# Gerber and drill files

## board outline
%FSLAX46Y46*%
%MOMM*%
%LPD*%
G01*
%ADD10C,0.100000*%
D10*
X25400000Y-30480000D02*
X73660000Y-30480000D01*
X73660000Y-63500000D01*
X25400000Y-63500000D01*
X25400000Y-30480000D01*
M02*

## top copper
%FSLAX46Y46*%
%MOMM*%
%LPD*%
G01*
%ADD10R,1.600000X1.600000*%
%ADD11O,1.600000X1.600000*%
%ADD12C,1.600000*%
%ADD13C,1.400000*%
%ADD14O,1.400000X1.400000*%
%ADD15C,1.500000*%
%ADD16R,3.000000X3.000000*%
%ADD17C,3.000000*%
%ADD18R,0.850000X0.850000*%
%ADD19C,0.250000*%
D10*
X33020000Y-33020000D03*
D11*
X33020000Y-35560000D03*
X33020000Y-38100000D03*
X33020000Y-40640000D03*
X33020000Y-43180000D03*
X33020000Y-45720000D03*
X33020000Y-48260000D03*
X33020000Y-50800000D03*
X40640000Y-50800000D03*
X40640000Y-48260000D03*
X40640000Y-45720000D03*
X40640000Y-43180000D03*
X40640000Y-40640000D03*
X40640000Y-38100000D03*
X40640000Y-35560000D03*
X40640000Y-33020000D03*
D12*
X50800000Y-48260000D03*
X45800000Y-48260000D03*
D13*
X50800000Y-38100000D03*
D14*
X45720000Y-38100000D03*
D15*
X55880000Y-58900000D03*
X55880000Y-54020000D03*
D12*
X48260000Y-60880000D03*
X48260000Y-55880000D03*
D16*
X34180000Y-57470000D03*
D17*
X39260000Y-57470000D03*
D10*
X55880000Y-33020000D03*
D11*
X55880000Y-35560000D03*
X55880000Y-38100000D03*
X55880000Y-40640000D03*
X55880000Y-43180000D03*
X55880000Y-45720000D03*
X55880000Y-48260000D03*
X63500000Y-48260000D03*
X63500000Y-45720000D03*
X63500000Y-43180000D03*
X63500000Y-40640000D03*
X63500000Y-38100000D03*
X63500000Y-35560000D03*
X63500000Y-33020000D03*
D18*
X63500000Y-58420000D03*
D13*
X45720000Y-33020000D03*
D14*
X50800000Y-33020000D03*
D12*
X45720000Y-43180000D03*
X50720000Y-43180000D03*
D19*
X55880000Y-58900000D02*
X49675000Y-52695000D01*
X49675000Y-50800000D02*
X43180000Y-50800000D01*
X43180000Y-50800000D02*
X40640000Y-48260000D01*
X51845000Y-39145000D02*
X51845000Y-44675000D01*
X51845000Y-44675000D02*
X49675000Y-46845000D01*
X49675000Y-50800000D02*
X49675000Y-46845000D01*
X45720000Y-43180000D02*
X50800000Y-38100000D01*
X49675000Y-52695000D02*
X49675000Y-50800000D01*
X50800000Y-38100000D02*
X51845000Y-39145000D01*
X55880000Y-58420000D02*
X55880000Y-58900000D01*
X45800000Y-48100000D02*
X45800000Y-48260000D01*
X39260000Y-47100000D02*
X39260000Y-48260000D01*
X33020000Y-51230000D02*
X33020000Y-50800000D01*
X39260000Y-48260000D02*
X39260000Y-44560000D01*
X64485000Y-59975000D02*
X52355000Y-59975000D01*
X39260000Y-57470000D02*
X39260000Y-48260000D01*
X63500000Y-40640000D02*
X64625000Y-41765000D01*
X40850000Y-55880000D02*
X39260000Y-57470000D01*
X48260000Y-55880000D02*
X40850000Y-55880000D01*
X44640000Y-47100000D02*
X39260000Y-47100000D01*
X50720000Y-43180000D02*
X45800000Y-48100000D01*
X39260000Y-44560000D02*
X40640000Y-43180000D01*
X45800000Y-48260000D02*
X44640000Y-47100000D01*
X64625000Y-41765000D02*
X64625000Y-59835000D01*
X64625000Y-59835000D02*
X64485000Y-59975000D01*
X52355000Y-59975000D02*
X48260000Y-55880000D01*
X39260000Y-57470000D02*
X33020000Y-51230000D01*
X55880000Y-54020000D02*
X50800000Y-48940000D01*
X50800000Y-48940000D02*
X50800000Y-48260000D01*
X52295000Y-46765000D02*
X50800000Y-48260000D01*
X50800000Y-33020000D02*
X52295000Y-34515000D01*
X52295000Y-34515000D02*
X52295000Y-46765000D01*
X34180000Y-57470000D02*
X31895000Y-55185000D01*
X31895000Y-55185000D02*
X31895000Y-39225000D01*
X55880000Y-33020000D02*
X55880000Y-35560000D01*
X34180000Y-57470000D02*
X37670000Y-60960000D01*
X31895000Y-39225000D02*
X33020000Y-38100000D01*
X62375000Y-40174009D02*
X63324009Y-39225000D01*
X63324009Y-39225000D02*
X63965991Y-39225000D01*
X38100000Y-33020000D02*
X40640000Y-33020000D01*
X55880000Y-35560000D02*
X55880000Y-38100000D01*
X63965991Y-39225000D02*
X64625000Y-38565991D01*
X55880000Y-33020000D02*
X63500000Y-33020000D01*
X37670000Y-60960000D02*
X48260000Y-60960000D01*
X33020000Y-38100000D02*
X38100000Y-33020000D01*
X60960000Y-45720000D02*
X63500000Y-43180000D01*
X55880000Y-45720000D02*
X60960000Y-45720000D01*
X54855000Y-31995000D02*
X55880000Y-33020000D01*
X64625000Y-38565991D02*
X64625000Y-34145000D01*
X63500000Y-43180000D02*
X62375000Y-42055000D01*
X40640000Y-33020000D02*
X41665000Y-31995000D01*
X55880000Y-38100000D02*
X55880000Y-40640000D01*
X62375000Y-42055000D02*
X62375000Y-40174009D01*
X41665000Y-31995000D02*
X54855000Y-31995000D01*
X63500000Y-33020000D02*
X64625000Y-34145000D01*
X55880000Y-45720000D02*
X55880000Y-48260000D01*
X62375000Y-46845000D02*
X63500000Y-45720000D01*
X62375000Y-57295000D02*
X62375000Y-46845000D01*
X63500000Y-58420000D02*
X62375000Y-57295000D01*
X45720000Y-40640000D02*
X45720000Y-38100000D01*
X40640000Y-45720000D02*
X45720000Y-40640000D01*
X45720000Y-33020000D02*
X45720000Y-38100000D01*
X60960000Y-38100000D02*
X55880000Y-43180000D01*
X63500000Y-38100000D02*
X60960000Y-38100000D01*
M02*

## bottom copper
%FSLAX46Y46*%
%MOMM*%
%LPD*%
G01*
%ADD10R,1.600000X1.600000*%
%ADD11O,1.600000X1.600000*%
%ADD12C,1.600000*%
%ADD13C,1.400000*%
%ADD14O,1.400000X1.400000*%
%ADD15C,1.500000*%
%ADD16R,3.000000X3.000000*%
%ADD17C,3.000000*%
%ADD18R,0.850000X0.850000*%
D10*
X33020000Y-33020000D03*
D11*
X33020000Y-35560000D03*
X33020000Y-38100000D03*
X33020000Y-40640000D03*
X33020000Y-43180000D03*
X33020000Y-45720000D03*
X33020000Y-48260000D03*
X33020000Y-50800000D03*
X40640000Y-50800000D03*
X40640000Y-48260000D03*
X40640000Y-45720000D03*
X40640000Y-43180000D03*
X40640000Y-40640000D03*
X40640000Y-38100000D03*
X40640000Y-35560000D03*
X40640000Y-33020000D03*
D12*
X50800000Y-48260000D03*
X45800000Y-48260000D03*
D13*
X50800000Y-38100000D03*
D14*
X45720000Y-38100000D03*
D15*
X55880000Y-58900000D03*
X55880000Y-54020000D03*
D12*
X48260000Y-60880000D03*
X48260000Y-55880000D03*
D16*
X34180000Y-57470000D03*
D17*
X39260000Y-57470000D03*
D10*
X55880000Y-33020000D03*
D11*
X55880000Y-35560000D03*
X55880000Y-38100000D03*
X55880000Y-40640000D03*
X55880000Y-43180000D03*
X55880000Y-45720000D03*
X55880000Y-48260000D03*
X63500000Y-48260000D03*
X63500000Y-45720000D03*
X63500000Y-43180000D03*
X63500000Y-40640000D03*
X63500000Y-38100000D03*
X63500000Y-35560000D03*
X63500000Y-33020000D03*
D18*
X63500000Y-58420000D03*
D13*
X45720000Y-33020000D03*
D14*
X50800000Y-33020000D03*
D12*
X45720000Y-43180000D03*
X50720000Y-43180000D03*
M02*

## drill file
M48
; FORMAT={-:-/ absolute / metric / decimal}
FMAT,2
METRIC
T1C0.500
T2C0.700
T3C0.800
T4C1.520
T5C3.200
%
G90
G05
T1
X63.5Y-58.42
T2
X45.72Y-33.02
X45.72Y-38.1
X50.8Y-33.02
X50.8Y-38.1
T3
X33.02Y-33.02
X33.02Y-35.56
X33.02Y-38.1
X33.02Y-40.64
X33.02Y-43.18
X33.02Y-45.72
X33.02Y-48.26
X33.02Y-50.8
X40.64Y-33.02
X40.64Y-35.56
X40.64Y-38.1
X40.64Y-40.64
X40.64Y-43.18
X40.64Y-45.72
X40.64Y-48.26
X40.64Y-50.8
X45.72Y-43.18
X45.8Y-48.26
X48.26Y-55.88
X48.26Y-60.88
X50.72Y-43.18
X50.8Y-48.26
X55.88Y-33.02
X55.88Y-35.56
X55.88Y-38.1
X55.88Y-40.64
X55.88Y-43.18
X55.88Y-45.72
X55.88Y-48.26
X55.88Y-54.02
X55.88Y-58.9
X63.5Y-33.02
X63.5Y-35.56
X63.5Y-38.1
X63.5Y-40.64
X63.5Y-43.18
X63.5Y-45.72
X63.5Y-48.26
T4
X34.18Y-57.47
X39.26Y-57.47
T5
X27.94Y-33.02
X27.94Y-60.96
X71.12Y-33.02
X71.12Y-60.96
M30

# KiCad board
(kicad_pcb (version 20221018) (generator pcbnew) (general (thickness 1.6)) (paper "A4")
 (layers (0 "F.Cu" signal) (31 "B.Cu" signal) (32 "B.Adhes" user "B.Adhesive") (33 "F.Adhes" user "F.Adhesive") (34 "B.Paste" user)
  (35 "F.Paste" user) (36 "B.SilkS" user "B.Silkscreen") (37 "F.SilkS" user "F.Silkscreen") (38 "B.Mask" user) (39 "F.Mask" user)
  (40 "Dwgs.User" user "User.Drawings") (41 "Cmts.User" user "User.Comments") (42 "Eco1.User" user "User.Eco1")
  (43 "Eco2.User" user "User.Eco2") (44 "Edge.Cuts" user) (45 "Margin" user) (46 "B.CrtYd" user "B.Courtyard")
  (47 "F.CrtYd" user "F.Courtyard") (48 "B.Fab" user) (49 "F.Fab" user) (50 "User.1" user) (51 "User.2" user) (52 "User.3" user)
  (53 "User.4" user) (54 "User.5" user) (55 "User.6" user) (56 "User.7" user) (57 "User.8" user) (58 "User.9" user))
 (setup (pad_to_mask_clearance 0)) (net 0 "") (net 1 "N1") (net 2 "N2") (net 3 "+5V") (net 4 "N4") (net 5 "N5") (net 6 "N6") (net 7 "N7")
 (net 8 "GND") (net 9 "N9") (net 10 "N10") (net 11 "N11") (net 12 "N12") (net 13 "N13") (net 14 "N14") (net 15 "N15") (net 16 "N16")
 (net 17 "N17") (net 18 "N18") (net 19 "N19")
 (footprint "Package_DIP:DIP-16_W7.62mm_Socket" (layer "F.Cu") (at 33.02 33.02)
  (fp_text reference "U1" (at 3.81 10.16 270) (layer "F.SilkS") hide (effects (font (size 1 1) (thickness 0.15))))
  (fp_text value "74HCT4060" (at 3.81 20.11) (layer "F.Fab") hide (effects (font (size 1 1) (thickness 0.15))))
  (pad "1" thru_hole rect (at 0 0) (size 1.6 1.6) (drill 0.8) (layers "*.Cu" "*.Mask") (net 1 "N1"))
  (pad "2" thru_hole oval (at 0 2.54) (size 1.6 1.6) (drill 0.8) (layers "*.Cu" "*.Mask") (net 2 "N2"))
  (pad "3" thru_hole oval (at 0 5.08) (size 1.6 1.6) (drill 0.8) (layers "*.Cu" "*.Mask") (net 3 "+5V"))
  (pad "4" thru_hole oval (at 0 7.62) (size 1.6 1.6) (drill 0.8) (layers "*.Cu" "*.Mask") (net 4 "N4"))
  (pad "5" thru_hole oval (at 0 10.16) (size 1.6 1.6) (drill 0.8) (layers "*.Cu" "*.Mask") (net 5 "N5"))
  (pad "6" thru_hole oval (at 0 12.7) (size 1.6 1.6) (drill 0.8) (layers "*.Cu" "*.Mask") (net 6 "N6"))
  (pad "7" thru_hole oval (at 0 15.24) (size 1.6 1.6) (drill 0.8) (layers "*.Cu" "*.Mask") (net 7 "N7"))
  (pad "8" thru_hole oval (at 0 17.78) (size 1.6 1.6) (drill 0.8) (layers "*.Cu" "*.Mask") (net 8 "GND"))
  (pad "9" thru_hole oval (at 7.62 17.78) (size 1.6 1.6) (drill 0.8) (layers "*.Cu" "*.Mask") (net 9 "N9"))
  (pad "10" thru_hole oval (at 7.62 15.24) (size 1.6 1.6) (drill 0.8) (layers "*.Cu" "*.Mask") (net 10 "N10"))
  (pad "11" thru_hole oval (at 7.62 12.7) (size 1.6 1.6) (drill 0.8) (layers "*.Cu" "*.Mask") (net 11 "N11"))
  (pad "12" thru_hole oval (at 7.62 10.16) (size 1.6 1.6) (drill 0.8) (layers "*.Cu" "*.Mask") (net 8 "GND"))
  (pad "13" thru_hole oval (at 7.62 7.62) (size 1.6 1.6) (drill 0.8) (layers "*.Cu" "*.Mask") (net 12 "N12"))
  (pad "14" thru_hole oval (at 7.62 5.08) (size 1.6 1.6) (drill 0.8) (layers "*.Cu" "*.Mask") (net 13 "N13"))
  (pad "15" thru_hole oval (at 7.62 2.54) (size 1.6 1.6) (drill 0.8) (layers "*.Cu" "*.Mask") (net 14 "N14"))
  (pad "16" thru_hole oval (at 7.62 0) (size 1.6 1.6) (drill 0.8) (layers "*.Cu" "*.Mask") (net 3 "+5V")))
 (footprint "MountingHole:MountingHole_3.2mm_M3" (layer "F.Cu") (at 71.12 60.96)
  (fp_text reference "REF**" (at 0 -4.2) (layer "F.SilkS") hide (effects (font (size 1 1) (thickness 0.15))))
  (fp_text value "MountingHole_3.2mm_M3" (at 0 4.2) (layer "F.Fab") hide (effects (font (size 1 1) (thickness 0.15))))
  (pad "" np_thru_hole circle (at 0 0) (size 3.2 3.2) (drill 3.2) (layers "*.Cu" "*.Mask")))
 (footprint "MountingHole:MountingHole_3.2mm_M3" (layer "F.Cu") (at 27.94 60.96)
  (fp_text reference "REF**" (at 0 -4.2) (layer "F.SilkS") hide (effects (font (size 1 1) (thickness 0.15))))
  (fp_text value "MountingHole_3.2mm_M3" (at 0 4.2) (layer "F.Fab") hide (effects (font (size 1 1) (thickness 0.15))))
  (pad "" np_thru_hole circle (at 0 0) (size 3.2 3.2) (drill 3.2) (layers "*.Cu" "*.Mask")))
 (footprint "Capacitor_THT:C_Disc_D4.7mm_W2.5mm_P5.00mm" (layer "F.Cu") (at 50.8 48.26 180)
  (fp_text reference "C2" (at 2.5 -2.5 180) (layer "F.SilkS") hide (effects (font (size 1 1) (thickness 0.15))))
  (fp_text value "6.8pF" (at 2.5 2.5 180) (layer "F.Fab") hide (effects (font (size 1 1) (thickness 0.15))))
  (pad "1" thru_hole circle (at 0 0 180) (size 1.6 1.6) (drill 0.8) (layers "*.Cu" "*.Mask") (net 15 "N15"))
  (pad "2" thru_hole circle (at 5 0 180) (size 1.6 1.6) (drill 0.8) (layers "*.Cu" "*.Mask") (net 8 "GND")))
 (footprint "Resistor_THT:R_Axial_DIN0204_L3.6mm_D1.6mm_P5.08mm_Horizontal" (layer "F.Cu") (at 50.8 38.1 180)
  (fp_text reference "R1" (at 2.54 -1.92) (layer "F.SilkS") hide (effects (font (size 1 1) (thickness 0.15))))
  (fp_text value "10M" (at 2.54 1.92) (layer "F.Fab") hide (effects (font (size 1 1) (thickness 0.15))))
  (pad "1" thru_hole circle (at 0 0 180) (size 1.4 1.4) (drill 0.7) (layers "*.Cu" "*.Mask") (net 10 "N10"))
  (pad "2" thru_hole oval (at 5.08 0 180) (size 1.4 1.4) (drill 0.7) (layers "*.Cu" "*.Mask") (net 11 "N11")))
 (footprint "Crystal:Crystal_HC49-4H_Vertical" (layer "F.Cu") (at 55.88 58.9 90)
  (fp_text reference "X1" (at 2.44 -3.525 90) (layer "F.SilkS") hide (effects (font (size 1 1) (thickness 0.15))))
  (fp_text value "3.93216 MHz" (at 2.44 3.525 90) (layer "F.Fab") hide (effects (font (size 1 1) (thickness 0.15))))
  (pad "1" thru_hole circle (at 0 0 90) (size 1.5 1.5) (drill 0.8) (layers "*.Cu" "*.Mask") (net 10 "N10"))
  (pad "2" thru_hole circle (at 4.88 0 90) (size 1.5 1.5) (drill 0.8) (layers "*.Cu" "*.Mask") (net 15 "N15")))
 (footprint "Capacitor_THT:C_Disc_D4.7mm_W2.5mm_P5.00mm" (layer "F.Cu") (at 48.26 60.88 90)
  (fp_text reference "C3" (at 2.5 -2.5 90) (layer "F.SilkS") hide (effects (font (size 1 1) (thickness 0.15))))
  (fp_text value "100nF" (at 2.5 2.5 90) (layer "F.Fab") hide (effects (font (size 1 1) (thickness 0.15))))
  (pad "1" thru_hole circle (at 0 0 90) (size 1.6 1.6) (drill 0.8) (layers "*.Cu" "*.Mask") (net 3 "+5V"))
  (pad "2" thru_hole circle (at 5 0 90) (size 1.6 1.6) (drill 0.8) (layers "*.Cu" "*.Mask") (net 8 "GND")))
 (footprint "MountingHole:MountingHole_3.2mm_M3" (layer "F.Cu") (at 71.12 33.02)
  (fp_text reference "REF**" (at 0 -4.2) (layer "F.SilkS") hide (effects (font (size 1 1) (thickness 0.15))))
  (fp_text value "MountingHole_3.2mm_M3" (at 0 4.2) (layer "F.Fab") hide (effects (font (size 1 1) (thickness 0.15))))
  (pad "" np_thru_hole circle (at 0 0) (size 3.2 3.2) (drill 3.2) (layers "*.Cu" "*.Mask")))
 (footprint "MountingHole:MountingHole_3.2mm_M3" (layer "F.Cu") (at 27.94 33.02)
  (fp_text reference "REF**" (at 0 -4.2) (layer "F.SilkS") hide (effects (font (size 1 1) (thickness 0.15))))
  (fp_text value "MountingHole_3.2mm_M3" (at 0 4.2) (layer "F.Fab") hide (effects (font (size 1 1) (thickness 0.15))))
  (pad "" np_thru_hole circle (at 0 0) (size 3.2 3.2) (drill 3.2) (layers "*.Cu" "*.Mask")))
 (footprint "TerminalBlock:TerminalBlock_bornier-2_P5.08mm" (layer "F.Cu") (at 34.18 57.47)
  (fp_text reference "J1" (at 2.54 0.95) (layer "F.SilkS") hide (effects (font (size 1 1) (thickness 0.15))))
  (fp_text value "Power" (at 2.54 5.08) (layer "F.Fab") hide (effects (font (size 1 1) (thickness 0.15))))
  (pad "1" thru_hole rect (at 0 0) (size 3 3) (drill 1.52) (layers "*.Cu" "*.Mask") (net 3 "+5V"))
  (pad "2" thru_hole circle (at 5.08 0) (size 3 3) (drill 1.52) (layers "*.Cu" "*.Mask") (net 8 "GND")))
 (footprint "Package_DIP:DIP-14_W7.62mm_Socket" (layer "F.Cu") (at 55.88 33.02)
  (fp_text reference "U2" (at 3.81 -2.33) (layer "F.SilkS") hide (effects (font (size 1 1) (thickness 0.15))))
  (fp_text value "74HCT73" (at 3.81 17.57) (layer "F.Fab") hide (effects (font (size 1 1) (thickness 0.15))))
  (pad "1" thru_hole rect (at 0 0) (size 1.6 1.6) (drill 0.8) (layers "*.Cu" "*.Mask") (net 3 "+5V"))
  (pad "2" thru_hole oval (at 0 2.54) (size 1.6 1.6) (drill 0.8) (layers "*.Cu" "*.Mask") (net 3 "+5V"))
  (pad "3" thru_hole oval (at 0 5.08) (size 1.6 1.6) (drill 0.8) (layers "*.Cu" "*.Mask") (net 3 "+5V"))
  (pad "4" thru_hole oval (at 0 7.62) (size 1.6 1.6) (drill 0.8) (layers "*.Cu" "*.Mask") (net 3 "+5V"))
  (pad "5" thru_hole oval (at 0 10.16) (size 1.6 1.6) (drill 0.8) (layers "*.Cu" "*.Mask") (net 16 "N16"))
  (pad "6" thru_hole oval (at 0 12.7) (size 1.6 1.6) (drill 0.8) (layers "*.Cu" "*.Mask") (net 3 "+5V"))
  (pad "7" thru_hole oval (at 0 15.24) (size 1.6 1.6) (drill 0.8) (layers "*.Cu" "*.Mask") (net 3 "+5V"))
  (pad "8" thru_hole oval (at 7.62 15.24) (size 1.6 1.6) (drill 0.8) (layers "*.Cu" "*.Mask") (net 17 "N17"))
  (pad "9" thru_hole oval (at 7.62 12.7) (size 1.6 1.6) (drill 0.8) (layers "*.Cu" "*.Mask") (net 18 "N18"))
  (pad "10" thru_hole oval (at 7.62 10.16) (size 1.6 1.6) (drill 0.8) (layers "*.Cu" "*.Mask") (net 3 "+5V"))
  (pad "11" thru_hole oval (at 7.62 7.62) (size 1.6 1.6) (drill 0.8) (layers "*.Cu" "*.Mask") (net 8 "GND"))
  (pad "12" thru_hole oval (at 7.62 5.08) (size 1.6 1.6) (drill 0.8) (layers "*.Cu" "*.Mask") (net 16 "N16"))
  (pad "13" thru_hole oval (at 7.62 2.54) (size 1.6 1.6) (drill 0.8) (layers "*.Cu" "*.Mask") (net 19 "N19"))
  (pad "14" thru_hole oval (at 7.62 0) (size 1.6 1.6) (drill 0.8) (layers "*.Cu" "*.Mask") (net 3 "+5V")))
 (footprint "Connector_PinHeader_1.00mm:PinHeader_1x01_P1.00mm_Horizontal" (layer "F.Cu") (at 63.5 58.42 -90)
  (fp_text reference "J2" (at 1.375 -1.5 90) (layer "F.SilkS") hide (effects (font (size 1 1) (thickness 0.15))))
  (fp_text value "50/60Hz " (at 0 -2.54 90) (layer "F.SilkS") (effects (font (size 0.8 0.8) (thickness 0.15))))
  (pad "1" thru_hole rect (at 0 0 270) (size 0.85 0.85) (drill 0.5) (layers "*.Cu" "*.Mask") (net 18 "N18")))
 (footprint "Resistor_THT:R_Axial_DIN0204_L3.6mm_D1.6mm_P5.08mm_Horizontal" (layer "F.Cu") (at 45.72 33.02)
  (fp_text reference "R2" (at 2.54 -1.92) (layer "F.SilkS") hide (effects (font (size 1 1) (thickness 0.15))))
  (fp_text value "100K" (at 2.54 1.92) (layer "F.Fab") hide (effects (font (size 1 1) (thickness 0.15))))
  (pad "1" thru_hole circle (at 0 0) (size 1.4 1.4) (drill 0.7) (layers "*.Cu" "*.Mask") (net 11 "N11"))
  (pad "2" thru_hole oval (at 5.08 0) (size 1.4 1.4) (drill 0.7) (layers "*.Cu" "*.Mask") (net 15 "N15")))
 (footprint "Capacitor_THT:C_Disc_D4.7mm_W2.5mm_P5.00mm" (layer "F.Cu") (at 45.72 43.18)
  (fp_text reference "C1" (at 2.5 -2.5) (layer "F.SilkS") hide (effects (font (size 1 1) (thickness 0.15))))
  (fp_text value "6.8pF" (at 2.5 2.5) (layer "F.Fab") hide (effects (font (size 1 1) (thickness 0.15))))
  (pad "1" thru_hole circle (at 0 0) (size 1.6 1.6) (drill 0.8) (layers "*.Cu" "*.Mask") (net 10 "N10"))
  (pad "2" thru_hole circle (at 5 0) (size 1.6 1.6) (drill 0.8) (layers "*.Cu" "*.Mask") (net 8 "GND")))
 (gr_rect (start 25.4 30.48) (end 73.66 63.5) (stroke (width 0.1) (type default)) (fill none) (layer "Edge.Cuts"))
 (segment (start 55.88 58.9) (end 49.675 52.695) (width 0.25) (layer "F.Cu") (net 10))
 (segment (start 49.675 50.8) (end 43.18 50.8) (width 0.25) (layer "F.Cu") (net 10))
 (segment (start 43.18 50.8) (end 40.64 48.26) (width 0.25) (layer "F.Cu") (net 10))
 (segment (start 51.845 39.145) (end 51.845 44.675) (width 0.25) (layer "F.Cu") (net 10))
 (segment (start 51.845 44.675) (end 49.675 46.845) (width 0.25) (layer "F.Cu") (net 10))
 (segment (start 49.675 50.8) (end 49.675 46.845) (width 0.25) (layer "F.Cu") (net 10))
 (segment (start 45.72 43.18) (end 50.8 38.1) (width 0.25) (layer "F.Cu") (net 10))
 (segment (start 49.675 52.695) (end 49.675 50.8) (width 0.25) (layer "F.Cu") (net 10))
 (segment (start 50.8 38.1) (end 51.845 39.145) (width 0.25) (layer "F.Cu") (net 10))
 (segment (start 55.88 58.42) (end 55.88 58.9) (width 0.25) (layer "F.Cu") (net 10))
 (segment (start 45.8 48.1) (end 45.8 48.26) (width 0.25) (layer "F.Cu") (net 8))
 (segment (start 39.26 47.1) (end 39.26 48.26) (width 0.25) (layer "F.Cu") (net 8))
 (segment (start 33.02 51.23) (end 33.02 50.8) (width 0.25) (layer "F.Cu") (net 8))
 (segment (start 39.26 48.26) (end 39.26 44.56) (width 0.25) (layer "F.Cu") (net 8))
 (segment (start 64.485 59.975) (end 52.355 59.975) (width 0.25) (layer "F.Cu") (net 8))
 (segment (start 39.26 57.47) (end 39.26 48.26) (width 0.25) (layer "F.Cu") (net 8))
 (segment (start 63.5 40.64) (end 64.625 41.765) (width 0.25) (layer "F.Cu") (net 8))
 (segment (start 40.85 55.88) (end 39.26 57.47) (width 0.25) (layer "F.Cu") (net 8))
 (segment (start 48.26 55.88) (end 40.85 55.88) (width 0.25) (layer "F.Cu") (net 8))
 (segment (start 44.64 47.1) (end 39.26 47.1) (width 0.25) (layer "F.Cu") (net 8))
 (segment (start 50.72 43.18) (end 45.8 48.1) (width 0.25) (layer "F.Cu") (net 8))
 (segment (start 39.26 44.56) (end 40.64 43.18) (width 0.25) (layer "F.Cu") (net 8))
 (segment (start 45.8 48.26) (end 44.64 47.1) (width 0.25) (layer "F.Cu") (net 8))
 (segment (start 64.625 41.765) (end 64.625 59.835) (width 0.25) (layer "F.Cu") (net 8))
 (segment (start 64.625 59.835) (end 64.485 59.975) (width 0.25) (layer "F.Cu") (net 8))
 (segment (start 52.355 59.975) (end 48.26 55.88) (width 0.25) (layer "F.Cu") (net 8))
 (segment (start 39.26 57.47) (end 33.02 51.23) (width 0.25) (layer "F.Cu") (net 8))
 (segment (start 55.88 54.02) (end 50.8 48.94) (width 0.25) (layer "F.Cu") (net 15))
 (segment (start 50.8 48.94) (end 50.8 48.26) (width 0.25) (layer "F.Cu") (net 15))
 (segment (start 52.295 46.765) (end 50.8 48.26) (width 0.25) (layer "F.Cu") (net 15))
 (segment (start 50.8 33.02) (end 52.295 34.515) (width 0.25) (layer "F.Cu") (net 15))
 (segment (start 52.295 34.515) (end 52.295 46.765) (width 0.25) (layer "F.Cu") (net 15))
 (segment (start 34.18 57.47) (end 31.895 55.185) (width 0.25) (layer "F.Cu") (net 3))
 (segment (start 31.895 55.185) (end 31.895 39.225) (width 0.25) (layer "F.Cu") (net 3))
 (segment (start 55.88 33.02) (end 55.88 35.56) (width 0.25) (layer "F.Cu") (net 3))
 (segment (start 34.18 57.47) (end 37.67 60.96) (width 0.25) (layer "F.Cu") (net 3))
 (segment (start 31.895 39.225) (end 33.02 38.1) (width 0.25) (layer "F.Cu") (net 3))
 (segment (start 62.375 40.174009) (end 63.324009 39.225) (width 0.25) (layer "F.Cu") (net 3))
 (segment (start 63.324009 39.225) (end 63.965991 39.225) (width 0.25) (layer "F.Cu") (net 3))
 (segment (start 38.1 33.02) (end 40.64 33.02) (width 0.25) (layer "F.Cu") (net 3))
 (segment (start 55.88 35.56) (end 55.88 38.1) (width 0.25) (layer "F.Cu") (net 3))
 (segment (start 63.965991 39.225) (end 64.625 38.565991) (width 0.25) (layer "F.Cu") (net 3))
 (segment (start 55.88 33.02) (end 63.5 33.02) (width 0.25) (layer "F.Cu") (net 3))
 (segment (start 37.67 60.96) (end 48.26 60.96) (width 0.25) (layer "F.Cu") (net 3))
 (segment (start 33.02 38.1) (end 38.1 33.02) (width 0.25) (layer "F.Cu") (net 3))
 (segment (start 60.96 45.72) (end 63.5 43.18) (width 0.25) (layer "F.Cu") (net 3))
 (segment (start 55.88 45.72) (end 60.96 45.72) (width 0.25) (layer "F.Cu") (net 3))
 (segment (start 54.855 31.995) (end 55.88 33.02) (width 0.25) (layer "F.Cu") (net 3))
 (segment (start 64.625 38.565991) (end 64.625 34.145) (width 0.25) (layer "F.Cu") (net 3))
 (segment (start 63.5 43.18) (end 62.375 42.055) (width 0.25) (layer "F.Cu") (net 3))
 (segment (start 40.64 33.02) (end 41.665 31.995) (width 0.25) (layer "F.Cu") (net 3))
 (segment (start 55.88 38.1) (end 55.88 40.64) (width 0.25) (layer "F.Cu") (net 3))
 (segment (start 62.375 42.055) (end 62.375 40.174009) (width 0.25) (layer "F.Cu") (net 3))
 (segment (start 41.665 31.995) (end 54.855 31.995) (width 0.25) (layer "F.Cu") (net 3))
 (segment (start 63.5 33.02) (end 64.625 34.145) (width 0.25) (layer "F.Cu") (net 3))
 (segment (start 55.88 45.72) (end 55.88 48.26) (width 0.25) (layer "F.Cu") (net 3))
 (segment (start 62.375 46.845) (end 63.5 45.72) (width 0.25) (layer "F.Cu") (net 18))
 (segment (start 62.375 57.295) (end 62.375 46.845) (width 0.25) (layer "F.Cu") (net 18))
 (segment (start 63.5 58.42) (end 62.375 57.295) (width 0.25) (layer "F.Cu") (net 18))
 (segment (start 45.72 40.64) (end 45.72 38.1) (width 0.25) (layer "F.Cu") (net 11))
 (segment (start 40.64 45.72) (end 45.72 40.64) (width 0.25) (layer "F.Cu") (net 11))
 (segment (start 45.72 33.02) (end 45.72 38.1) (width 0.25) (layer "F.Cu") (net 11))
 (segment (start 60.96 38.1) (end 55.88 43.18) (width 0.25) (layer "F.Cu") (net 16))
 (segment (start 63.5 38.1) (end 60.96 38.1) (width 0.25) (layer "F.Cu") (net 16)))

